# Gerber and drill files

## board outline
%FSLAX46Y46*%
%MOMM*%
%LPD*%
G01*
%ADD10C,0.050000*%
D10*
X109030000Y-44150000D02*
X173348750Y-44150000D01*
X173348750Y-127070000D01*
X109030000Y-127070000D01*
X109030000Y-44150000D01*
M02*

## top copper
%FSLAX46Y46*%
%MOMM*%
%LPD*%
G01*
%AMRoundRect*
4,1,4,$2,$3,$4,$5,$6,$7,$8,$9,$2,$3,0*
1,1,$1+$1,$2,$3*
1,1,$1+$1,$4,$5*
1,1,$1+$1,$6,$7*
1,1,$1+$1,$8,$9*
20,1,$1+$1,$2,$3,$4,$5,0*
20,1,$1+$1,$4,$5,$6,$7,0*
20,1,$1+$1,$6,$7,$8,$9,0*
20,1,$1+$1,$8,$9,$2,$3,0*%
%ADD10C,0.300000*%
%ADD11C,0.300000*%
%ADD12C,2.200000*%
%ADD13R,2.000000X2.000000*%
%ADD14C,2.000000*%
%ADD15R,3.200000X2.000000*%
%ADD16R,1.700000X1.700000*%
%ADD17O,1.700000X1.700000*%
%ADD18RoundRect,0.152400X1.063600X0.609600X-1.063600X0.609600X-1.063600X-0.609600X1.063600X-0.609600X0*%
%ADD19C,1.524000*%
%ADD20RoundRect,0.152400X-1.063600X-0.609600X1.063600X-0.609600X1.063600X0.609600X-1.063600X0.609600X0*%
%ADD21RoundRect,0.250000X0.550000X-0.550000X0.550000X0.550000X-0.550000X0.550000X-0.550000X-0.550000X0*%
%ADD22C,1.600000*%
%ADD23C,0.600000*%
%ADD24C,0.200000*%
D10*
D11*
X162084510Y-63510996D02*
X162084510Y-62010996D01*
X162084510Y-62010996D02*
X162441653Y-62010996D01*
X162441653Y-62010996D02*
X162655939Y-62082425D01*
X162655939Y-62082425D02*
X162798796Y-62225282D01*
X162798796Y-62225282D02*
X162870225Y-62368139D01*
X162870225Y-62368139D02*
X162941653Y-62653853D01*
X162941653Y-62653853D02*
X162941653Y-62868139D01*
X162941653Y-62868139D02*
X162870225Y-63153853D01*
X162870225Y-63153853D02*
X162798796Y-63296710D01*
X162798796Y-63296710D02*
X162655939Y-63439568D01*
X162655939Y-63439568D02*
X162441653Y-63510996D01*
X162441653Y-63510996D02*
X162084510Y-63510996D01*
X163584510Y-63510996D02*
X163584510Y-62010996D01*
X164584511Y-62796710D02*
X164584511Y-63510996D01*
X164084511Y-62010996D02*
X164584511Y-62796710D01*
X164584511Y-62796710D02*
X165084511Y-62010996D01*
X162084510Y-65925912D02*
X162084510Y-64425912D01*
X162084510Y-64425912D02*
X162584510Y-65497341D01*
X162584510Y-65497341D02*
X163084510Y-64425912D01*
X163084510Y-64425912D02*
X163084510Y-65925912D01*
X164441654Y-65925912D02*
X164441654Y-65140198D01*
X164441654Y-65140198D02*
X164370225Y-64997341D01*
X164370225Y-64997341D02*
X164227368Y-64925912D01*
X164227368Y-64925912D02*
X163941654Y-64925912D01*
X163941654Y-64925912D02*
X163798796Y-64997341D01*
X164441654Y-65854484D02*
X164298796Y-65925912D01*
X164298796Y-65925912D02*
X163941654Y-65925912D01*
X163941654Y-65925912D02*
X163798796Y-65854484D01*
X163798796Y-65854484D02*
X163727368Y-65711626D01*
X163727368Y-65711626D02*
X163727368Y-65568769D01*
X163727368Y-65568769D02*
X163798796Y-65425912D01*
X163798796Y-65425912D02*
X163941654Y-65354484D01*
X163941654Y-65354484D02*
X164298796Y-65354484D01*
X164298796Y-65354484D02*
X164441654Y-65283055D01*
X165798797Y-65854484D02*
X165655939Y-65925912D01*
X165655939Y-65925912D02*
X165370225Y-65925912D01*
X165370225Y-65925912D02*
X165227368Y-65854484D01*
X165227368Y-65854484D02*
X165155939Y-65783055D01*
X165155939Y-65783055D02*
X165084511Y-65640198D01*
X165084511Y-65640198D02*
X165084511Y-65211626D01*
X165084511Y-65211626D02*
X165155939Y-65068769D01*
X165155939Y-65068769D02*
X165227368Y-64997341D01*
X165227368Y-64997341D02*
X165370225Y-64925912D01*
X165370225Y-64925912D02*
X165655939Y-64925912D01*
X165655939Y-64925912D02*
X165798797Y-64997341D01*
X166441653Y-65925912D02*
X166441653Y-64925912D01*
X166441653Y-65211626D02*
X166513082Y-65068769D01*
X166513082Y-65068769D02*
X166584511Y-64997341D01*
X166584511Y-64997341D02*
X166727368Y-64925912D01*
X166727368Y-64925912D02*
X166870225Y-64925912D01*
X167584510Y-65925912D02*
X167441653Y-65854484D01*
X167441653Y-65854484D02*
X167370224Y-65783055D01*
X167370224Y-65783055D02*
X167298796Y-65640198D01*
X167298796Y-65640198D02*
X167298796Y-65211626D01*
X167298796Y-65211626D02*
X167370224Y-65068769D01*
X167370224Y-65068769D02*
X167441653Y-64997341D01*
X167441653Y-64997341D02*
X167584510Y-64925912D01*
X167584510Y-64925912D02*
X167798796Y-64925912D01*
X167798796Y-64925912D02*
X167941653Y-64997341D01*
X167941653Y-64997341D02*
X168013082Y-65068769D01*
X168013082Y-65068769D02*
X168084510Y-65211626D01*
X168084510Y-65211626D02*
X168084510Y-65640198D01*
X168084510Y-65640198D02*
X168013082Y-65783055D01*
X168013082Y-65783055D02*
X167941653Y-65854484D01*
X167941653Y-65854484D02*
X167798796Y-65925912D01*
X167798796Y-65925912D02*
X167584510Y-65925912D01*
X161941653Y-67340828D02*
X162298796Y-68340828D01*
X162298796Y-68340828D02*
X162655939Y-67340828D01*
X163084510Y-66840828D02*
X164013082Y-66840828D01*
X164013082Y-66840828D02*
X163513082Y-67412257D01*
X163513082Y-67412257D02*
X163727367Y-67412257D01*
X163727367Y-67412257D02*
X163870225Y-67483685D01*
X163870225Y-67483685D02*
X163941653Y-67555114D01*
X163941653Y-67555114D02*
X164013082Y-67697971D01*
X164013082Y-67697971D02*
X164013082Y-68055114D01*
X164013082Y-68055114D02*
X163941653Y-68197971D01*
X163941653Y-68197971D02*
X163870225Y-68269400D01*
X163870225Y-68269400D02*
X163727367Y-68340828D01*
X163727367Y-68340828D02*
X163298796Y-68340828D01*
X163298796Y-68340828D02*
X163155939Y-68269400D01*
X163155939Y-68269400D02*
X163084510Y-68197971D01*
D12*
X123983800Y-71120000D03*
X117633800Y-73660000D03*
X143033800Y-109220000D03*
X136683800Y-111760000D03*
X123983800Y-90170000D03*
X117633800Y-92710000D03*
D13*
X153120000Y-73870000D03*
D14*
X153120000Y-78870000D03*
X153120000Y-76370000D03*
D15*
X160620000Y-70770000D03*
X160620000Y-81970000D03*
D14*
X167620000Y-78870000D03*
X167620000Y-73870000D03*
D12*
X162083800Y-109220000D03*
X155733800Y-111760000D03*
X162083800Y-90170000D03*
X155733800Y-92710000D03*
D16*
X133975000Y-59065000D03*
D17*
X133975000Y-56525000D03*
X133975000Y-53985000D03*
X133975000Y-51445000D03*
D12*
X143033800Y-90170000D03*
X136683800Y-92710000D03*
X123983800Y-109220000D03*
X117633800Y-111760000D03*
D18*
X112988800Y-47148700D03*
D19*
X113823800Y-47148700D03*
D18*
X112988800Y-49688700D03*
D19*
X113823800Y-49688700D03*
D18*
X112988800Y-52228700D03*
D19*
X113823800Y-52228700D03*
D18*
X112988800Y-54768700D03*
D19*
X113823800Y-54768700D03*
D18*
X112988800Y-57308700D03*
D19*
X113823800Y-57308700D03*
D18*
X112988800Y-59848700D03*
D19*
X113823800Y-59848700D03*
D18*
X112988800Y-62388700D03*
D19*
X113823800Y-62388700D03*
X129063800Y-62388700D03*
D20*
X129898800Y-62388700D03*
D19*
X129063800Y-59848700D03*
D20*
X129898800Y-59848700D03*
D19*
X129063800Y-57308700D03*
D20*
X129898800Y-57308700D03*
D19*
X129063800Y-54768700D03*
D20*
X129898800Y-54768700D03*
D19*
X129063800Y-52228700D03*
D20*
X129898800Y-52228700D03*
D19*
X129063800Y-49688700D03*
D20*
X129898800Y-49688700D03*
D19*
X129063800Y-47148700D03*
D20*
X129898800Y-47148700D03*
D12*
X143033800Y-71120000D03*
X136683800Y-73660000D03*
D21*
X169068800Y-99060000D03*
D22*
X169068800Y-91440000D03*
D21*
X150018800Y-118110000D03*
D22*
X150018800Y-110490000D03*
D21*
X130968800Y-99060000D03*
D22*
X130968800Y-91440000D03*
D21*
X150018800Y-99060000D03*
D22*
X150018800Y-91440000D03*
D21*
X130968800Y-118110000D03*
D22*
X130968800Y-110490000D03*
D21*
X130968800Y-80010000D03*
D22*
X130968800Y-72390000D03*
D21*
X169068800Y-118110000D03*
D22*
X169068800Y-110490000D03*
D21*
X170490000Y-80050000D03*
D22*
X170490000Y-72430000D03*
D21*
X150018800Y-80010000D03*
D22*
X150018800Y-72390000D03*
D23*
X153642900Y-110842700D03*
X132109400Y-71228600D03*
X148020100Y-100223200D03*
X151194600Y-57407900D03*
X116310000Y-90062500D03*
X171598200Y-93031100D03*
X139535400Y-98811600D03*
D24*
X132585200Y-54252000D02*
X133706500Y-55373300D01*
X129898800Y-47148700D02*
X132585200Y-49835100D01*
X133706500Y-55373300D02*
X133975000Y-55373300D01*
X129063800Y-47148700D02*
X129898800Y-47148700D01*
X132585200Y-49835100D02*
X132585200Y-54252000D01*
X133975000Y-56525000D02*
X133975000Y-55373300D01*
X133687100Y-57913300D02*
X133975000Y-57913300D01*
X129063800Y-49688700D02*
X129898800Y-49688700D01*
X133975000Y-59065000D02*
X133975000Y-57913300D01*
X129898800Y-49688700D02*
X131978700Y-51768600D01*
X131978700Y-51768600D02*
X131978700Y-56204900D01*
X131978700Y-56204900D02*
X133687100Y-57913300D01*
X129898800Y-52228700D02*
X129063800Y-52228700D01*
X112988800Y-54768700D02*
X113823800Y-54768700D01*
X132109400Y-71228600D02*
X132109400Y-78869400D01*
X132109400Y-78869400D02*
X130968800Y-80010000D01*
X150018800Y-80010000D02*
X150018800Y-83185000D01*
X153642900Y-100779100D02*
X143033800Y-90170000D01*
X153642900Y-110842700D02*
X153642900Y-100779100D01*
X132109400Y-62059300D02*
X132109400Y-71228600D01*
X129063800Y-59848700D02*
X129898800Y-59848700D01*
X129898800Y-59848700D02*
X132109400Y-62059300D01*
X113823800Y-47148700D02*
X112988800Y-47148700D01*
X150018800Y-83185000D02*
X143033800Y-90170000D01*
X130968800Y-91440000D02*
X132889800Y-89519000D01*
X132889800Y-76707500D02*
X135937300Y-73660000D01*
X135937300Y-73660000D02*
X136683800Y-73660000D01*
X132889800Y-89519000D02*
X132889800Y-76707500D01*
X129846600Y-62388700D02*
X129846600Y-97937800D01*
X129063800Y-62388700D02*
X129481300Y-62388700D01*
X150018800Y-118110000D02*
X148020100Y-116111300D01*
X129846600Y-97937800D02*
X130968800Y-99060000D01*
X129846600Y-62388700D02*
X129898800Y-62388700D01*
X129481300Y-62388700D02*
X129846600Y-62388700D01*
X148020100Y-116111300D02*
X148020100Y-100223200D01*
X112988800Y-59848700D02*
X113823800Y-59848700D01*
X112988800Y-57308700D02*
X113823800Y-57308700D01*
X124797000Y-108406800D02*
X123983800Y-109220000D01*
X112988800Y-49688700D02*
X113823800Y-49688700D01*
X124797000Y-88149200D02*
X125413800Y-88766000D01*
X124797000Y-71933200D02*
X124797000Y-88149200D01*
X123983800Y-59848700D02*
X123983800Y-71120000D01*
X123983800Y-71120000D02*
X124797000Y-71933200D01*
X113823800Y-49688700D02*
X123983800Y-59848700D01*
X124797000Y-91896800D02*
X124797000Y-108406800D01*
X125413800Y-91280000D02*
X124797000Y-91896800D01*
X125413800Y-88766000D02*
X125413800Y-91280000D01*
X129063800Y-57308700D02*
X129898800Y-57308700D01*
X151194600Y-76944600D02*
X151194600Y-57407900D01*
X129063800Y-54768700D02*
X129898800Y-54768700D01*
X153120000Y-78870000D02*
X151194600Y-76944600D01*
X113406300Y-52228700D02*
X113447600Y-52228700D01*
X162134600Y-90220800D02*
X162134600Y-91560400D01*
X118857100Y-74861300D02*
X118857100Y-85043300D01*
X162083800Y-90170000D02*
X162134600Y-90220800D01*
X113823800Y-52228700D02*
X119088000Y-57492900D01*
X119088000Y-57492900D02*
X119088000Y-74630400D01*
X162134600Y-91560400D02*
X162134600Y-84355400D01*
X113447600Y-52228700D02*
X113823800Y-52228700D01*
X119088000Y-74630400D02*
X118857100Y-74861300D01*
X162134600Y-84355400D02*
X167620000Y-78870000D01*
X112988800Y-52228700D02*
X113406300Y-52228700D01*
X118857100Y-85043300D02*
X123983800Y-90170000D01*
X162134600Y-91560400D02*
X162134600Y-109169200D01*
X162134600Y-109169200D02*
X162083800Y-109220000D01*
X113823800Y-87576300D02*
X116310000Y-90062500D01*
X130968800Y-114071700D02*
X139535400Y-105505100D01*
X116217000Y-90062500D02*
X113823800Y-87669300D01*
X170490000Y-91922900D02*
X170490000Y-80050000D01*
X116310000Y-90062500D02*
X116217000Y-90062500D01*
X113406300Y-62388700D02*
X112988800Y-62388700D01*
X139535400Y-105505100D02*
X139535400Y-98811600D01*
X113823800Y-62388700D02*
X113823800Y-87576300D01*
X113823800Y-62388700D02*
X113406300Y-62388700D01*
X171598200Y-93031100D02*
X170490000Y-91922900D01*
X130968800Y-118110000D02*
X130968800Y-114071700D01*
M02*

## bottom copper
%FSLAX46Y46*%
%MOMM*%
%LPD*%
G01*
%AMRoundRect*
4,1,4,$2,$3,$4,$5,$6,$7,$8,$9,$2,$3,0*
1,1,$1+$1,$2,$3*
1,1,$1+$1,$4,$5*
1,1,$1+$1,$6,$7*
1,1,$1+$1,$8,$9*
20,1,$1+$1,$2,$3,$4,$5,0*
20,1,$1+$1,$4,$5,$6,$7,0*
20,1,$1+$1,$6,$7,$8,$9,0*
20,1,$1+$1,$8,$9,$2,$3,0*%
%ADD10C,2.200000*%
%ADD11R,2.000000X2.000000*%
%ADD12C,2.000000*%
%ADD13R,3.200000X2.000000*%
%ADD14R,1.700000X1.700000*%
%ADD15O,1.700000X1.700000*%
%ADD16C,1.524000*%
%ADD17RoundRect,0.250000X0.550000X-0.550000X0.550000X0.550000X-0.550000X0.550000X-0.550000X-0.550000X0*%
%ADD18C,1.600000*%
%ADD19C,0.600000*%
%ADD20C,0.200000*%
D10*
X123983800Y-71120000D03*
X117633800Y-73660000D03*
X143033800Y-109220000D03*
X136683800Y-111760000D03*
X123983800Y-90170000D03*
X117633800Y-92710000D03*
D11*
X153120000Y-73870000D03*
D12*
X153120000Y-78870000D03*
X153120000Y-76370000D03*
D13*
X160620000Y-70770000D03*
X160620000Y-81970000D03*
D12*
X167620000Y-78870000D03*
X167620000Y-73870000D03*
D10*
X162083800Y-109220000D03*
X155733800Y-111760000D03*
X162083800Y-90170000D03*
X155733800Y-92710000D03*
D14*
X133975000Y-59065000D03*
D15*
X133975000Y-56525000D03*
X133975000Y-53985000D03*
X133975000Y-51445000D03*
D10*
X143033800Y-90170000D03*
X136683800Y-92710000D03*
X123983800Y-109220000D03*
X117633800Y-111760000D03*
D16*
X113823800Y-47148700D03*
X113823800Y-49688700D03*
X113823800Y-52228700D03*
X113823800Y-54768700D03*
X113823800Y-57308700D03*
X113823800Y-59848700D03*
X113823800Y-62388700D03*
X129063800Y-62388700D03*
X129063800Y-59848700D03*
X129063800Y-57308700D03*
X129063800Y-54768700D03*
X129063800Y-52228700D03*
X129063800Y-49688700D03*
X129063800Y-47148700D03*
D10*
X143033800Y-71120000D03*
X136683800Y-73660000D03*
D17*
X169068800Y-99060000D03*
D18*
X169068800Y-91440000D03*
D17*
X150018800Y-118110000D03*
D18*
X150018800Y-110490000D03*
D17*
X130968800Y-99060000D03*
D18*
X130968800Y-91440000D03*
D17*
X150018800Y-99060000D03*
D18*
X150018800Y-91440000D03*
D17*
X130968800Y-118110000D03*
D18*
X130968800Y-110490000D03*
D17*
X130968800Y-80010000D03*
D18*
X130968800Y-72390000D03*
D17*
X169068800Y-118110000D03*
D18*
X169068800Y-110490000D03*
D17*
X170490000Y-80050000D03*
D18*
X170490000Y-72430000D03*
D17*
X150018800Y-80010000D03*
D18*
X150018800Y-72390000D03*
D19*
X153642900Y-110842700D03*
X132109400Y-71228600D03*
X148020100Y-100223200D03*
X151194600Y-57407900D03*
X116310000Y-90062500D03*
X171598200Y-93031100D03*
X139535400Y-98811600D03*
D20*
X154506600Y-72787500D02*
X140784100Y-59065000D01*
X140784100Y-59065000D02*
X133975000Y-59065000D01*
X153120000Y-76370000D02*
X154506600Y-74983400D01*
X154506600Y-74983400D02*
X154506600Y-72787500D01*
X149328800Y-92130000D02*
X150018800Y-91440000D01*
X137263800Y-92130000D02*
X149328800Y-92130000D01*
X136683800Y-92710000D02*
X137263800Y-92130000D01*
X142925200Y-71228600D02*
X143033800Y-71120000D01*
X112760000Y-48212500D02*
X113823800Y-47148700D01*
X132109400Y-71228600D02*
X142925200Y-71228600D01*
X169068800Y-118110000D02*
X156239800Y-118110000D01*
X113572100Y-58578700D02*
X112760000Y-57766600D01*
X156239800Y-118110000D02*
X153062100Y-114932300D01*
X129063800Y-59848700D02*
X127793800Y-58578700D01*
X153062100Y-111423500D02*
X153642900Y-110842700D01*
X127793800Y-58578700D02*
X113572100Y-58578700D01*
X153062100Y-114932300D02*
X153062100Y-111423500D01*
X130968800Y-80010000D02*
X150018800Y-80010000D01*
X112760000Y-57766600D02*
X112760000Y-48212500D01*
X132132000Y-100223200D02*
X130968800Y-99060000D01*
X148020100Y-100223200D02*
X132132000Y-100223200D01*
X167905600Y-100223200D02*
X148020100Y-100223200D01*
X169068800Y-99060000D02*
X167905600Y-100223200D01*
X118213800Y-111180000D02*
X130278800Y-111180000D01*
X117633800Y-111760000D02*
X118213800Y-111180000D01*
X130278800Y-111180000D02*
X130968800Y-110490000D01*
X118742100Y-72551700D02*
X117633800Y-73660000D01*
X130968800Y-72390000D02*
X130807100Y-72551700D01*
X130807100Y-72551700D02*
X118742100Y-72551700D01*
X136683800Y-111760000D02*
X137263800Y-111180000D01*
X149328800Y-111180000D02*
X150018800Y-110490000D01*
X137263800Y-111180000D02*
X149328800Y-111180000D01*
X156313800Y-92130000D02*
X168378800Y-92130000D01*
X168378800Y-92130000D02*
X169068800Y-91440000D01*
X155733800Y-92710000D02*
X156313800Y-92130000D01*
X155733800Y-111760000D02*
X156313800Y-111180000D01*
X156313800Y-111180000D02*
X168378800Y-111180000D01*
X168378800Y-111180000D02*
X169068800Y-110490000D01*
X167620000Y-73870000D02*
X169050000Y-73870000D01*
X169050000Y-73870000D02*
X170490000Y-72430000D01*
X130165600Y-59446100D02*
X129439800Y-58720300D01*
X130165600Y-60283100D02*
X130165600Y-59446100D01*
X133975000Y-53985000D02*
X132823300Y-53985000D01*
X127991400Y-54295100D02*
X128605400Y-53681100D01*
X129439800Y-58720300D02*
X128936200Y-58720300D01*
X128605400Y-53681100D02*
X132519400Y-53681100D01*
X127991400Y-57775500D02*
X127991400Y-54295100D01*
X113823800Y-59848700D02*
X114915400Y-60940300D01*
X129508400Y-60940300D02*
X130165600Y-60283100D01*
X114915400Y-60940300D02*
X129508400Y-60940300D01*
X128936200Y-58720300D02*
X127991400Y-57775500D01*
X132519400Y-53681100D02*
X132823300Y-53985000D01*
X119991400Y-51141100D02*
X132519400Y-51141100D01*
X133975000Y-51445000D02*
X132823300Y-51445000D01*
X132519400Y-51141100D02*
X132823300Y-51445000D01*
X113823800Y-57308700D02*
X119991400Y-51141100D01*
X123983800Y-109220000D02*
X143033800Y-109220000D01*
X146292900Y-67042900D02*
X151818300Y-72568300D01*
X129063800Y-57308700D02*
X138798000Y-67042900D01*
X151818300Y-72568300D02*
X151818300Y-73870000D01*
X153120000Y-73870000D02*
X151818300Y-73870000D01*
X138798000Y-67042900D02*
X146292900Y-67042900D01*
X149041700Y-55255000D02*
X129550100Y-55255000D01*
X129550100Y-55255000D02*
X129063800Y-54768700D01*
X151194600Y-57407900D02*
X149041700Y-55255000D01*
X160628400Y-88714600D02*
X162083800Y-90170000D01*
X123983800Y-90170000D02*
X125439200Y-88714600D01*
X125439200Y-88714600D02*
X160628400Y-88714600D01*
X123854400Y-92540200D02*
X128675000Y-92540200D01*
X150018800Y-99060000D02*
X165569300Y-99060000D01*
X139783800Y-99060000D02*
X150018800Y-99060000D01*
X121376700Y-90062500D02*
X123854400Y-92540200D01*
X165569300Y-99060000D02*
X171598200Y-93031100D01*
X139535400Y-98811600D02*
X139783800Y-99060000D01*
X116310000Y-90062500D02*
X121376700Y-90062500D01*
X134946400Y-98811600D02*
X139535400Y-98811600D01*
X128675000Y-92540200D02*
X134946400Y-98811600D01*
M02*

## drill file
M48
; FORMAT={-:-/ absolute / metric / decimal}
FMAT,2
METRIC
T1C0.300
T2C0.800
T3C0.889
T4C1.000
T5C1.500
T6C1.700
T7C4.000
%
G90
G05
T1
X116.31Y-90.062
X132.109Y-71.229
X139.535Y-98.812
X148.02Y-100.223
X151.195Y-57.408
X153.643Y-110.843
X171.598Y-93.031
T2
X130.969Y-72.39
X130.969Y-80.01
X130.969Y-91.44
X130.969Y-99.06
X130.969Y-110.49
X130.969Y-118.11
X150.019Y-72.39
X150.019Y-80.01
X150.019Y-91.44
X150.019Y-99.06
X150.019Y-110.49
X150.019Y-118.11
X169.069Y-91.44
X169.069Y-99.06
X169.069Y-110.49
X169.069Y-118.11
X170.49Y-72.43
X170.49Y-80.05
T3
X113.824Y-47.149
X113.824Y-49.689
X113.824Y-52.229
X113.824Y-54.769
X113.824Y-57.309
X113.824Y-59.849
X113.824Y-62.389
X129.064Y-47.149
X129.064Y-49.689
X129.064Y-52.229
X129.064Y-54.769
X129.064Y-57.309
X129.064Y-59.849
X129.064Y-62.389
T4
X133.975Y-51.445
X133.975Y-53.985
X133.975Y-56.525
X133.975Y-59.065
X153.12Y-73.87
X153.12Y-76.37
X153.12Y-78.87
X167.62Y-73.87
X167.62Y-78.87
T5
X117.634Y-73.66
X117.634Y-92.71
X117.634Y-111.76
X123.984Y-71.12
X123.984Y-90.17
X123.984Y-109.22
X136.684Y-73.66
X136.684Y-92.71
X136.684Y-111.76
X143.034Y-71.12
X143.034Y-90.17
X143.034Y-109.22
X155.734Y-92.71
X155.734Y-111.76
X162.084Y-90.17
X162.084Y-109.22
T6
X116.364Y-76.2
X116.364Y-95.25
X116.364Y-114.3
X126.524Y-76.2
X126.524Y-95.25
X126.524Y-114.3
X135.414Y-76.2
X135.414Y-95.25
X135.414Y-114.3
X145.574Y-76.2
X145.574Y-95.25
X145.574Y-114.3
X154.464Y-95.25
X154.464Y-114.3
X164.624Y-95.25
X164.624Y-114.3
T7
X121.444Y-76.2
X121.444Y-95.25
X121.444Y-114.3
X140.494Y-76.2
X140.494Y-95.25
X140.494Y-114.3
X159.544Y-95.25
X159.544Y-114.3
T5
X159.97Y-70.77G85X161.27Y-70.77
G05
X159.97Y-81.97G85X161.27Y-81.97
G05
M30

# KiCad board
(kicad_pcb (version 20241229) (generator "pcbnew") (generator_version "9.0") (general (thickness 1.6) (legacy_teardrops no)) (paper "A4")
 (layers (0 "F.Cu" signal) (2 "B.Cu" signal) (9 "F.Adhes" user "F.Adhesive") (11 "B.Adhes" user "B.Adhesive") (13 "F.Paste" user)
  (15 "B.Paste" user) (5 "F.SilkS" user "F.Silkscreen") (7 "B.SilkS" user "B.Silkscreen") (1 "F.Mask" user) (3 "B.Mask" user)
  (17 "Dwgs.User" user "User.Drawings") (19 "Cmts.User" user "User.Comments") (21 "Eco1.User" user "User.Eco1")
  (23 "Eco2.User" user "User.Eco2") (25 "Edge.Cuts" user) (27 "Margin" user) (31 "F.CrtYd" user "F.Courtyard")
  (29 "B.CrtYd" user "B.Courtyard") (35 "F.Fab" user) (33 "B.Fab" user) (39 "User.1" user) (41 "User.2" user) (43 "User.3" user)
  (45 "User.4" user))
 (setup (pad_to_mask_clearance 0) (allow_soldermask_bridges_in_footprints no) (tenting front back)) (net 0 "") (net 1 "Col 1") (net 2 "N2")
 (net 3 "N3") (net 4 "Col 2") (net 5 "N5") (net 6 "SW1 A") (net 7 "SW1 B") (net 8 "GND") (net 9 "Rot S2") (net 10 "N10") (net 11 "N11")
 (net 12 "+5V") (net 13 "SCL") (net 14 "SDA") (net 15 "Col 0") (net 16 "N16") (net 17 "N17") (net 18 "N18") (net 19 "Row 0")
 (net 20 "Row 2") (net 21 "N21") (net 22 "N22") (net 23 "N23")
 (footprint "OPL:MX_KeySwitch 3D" (layer "F.Cu") (at 123.9838 71.12)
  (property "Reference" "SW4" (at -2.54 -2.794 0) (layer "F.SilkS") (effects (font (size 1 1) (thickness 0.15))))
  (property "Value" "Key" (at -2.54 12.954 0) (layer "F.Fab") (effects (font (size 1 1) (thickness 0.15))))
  (pad "" np_thru_hole circle (at -7.62 5.08) (size 1.7 1.7) (drill 1.7) (layers "*.Cu" "*.Mask"))
  (pad "" np_thru_hole circle (at -2.54 5.08) (size 4 4) (drill 4) (layers "*.Cu" "*.Mask"))
  (pad "" np_thru_hole circle (at 2.54 5.08) (size 1.7 1.7) (drill 1.7) (layers "*.Cu" "*.Mask"))
  (pad "1" thru_hole circle (at 0 0) (size 2.2 2.2) (drill 1.5) (layers "*.Cu" "*.Mask") (remove_unused_layers no) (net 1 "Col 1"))
  (pad "2" thru_hole circle (at -6.35 2.54) (size 2.2 2.2) (drill 1.5) (layers "*.Cu" "*.Mask") (remove_unused_layers no) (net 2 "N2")))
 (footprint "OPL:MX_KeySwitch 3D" (layer "F.Cu") (at 143.0338 109.22)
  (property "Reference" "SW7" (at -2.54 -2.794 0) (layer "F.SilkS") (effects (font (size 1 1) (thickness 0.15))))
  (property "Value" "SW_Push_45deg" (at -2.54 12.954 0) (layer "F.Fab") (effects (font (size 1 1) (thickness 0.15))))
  (pad "" np_thru_hole circle (at -7.62 5.08) (size 1.7 1.7) (drill 1.7) (layers "*.Cu" "*.Mask"))
  (pad "" np_thru_hole circle (at -2.54 5.08) (size 4 4) (drill 4) (layers "*.Cu" "*.Mask"))
  (pad "" np_thru_hole circle (at 2.54 5.08) (size 1.7 1.7) (drill 1.7) (layers "*.Cu" "*.Mask"))
  (pad "1" thru_hole circle (at 0 0) (size 2.2 2.2) (drill 1.5) (layers "*.Cu" "*.Mask") (remove_unused_layers no) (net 1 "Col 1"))
  (pad "2" thru_hole circle (at -6.35 2.54) (size 2.2 2.2) (drill 1.5) (layers "*.Cu" "*.Mask") (remove_unused_layers no) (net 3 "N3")))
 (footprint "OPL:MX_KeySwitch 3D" (layer "F.Cu") (at 123.9838 90.17)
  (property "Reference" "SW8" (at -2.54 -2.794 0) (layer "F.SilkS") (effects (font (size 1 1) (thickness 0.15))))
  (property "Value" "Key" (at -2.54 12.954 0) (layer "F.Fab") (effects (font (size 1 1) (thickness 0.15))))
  (pad "" np_thru_hole circle (at -7.62 5.08) (size 1.7 1.7) (drill 1.7) (layers "*.Cu" "*.Mask"))
  (pad "" np_thru_hole circle (at -2.54 5.08) (size 4 4) (drill 4) (layers "*.Cu" "*.Mask"))
  (pad "" np_thru_hole circle (at 2.54 5.08) (size 1.7 1.7) (drill 1.7) (layers "*.Cu" "*.Mask"))
  (pad "1" thru_hole circle (at 0 0) (size 2.2 2.2) (drill 1.5) (layers "*.Cu" "*.Mask") (remove_unused_layers no) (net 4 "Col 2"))
  (pad "2" thru_hole circle (at -6.35 2.54) (size 2.2 2.2) (drill 1.5) (layers "*.Cu" "*.Mask") (remove_unused_layers no) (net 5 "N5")))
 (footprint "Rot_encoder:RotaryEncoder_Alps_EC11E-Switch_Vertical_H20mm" (layer "F.Cu") (at 153.12 73.87)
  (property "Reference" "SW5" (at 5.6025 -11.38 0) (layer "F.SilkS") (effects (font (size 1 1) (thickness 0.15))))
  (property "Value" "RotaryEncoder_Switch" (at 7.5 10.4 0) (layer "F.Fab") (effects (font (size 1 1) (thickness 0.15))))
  (pad "A" thru_hole rect (at 0 0) (size 2 2) (drill 1) (layers "*.Cu" "*.Mask") (remove_unused_layers no) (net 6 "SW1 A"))
  (pad "B" thru_hole circle (at 0 5) (size 2 2) (drill 1) (layers "*.Cu" "*.Mask") (remove_unused_layers no) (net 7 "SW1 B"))
  (pad "C" thru_hole circle (at 0 2.5) (size 2 2) (drill 1) (layers "*.Cu" "*.Mask") (remove_unused_layers no) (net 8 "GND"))
  (pad "MP" thru_hole rect (at 7.5 -3.1) (size 3.2 2) (drill oval 2.8 1.5) (layers "*.Cu" "*.Mask") (remove_unused_layers no))
  (pad "MP" thru_hole rect (at 7.5 8.1) (size 3.2 2) (drill oval 2.8 1.5) (layers "*.Cu" "*.Mask") (remove_unused_layers no))
  (pad "S1" thru_hole circle (at 14.5 5) (size 2 2) (drill 1) (layers "*.Cu" "*.Mask") (remove_unused_layers no) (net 4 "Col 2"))
  (pad "S2" thru_hole circle (at 14.5 0) (size 2 2) (drill 1) (layers "*.Cu" "*.Mask") (remove_unused_layers no) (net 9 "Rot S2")))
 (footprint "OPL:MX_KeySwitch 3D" (layer "F.Cu") (at 162.0838 109.22)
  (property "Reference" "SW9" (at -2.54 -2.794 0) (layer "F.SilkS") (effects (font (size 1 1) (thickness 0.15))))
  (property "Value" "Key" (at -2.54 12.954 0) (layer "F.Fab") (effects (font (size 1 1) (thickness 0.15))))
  (pad "" np_thru_hole circle (at -7.62 5.08) (size 1.7 1.7) (drill 1.7) (layers "*.Cu" "*.Mask"))
  (pad "" np_thru_hole circle (at -2.54 5.08) (size 4 4) (drill 4) (layers "*.Cu" "*.Mask"))
  (pad "" np_thru_hole circle (at 2.54 5.08) (size 1.7 1.7) (drill 1.7) (layers "*.Cu" "*.Mask"))
  (pad "1" thru_hole circle (at 0 0) (size 2.2 2.2) (drill 1.5) (layers "*.Cu" "*.Mask") (remove_unused_layers no) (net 4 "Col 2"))
  (pad "2" thru_hole circle (at -6.35 2.54) (size 2.2 2.2) (drill 1.5) (layers "*.Cu" "*.Mask") (remove_unused_layers no) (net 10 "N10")))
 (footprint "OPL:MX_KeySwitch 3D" (layer "F.Cu") (at 162.0838 90.17)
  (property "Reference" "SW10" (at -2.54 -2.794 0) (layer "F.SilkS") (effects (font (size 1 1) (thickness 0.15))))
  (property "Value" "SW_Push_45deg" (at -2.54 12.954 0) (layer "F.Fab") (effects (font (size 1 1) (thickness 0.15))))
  (pad "" np_thru_hole circle (at -7.62 5.08) (size 1.7 1.7) (drill 1.7) (layers "*.Cu" "*.Mask"))
  (pad "" np_thru_hole circle (at -2.54 5.08) (size 4 4) (drill 4) (layers "*.Cu" "*.Mask"))
  (pad "" np_thru_hole circle (at 2.54 5.08) (size 1.7 1.7) (drill 1.7) (layers "*.Cu" "*.Mask"))
  (pad "1" thru_hole circle (at 0 0) (size 2.2 2.2) (drill 1.5) (layers "*.Cu" "*.Mask") (remove_unused_layers no) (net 4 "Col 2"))
  (pad "2" thru_hole circle (at -6.35 2.54) (size 2.2 2.2) (drill 1.5) (layers "*.Cu" "*.Mask") (remove_unused_layers no) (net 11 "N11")))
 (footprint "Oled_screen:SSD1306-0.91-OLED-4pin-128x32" (layer "F.Cu") (at 170.475 61.255 180)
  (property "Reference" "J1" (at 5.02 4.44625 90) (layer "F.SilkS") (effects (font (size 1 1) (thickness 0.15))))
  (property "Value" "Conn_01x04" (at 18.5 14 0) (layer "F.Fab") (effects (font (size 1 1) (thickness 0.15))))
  (pad "1" thru_hole rect (at 36.5 2.19 180) (size 1.7 1.7) (drill 1) (layers "*.Cu" "*.Mask") (remove_unused_layers no) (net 8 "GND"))
  (pad "2" thru_hole oval (at 36.5 4.73 180) (size 1.7 1.7) (drill 1) (layers "*.Cu" "*.Mask") (remove_unused_layers no) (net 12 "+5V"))
  (pad "3" thru_hole oval (at 36.5 7.27 180) (size 1.7 1.7) (drill 1) (layers "*.Cu" "*.Mask") (remove_unused_layers no) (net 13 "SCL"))
  (pad "4" thru_hole oval (at 36.5 9.81 180) (size 1.7 1.7) (drill 1) (layers "*.Cu" "*.Mask") (remove_unused_layers no) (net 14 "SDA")))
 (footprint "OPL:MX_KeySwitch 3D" (layer "F.Cu") (at 143.0338 90.17)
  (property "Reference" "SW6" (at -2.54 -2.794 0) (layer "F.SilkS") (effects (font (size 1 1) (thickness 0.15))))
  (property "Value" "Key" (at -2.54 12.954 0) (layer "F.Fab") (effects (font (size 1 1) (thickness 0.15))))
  (pad "" np_thru_hole circle (at -7.62 5.08) (size 1.7 1.7) (drill 1.7) (layers "*.Cu" "*.Mask"))
  (pad "" np_thru_hole circle (at -2.54 5.08) (size 4 4) (drill 4) (layers "*.Cu" "*.Mask"))
  (pad "" np_thru_hole circle (at 2.54 5.08) (size 1.7 1.7) (drill 1.7) (layers "*.Cu" "*.Mask"))
  (pad "1" thru_hole circle (at 0 0) (size 2.2 2.2) (drill 1.5) (layers "*.Cu" "*.Mask") (remove_unused_layers no) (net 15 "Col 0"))
  (pad "2" thru_hole circle (at -6.35 2.54) (size 2.2 2.2) (drill 1.5) (layers "*.Cu" "*.Mask") (remove_unused_layers no) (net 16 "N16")))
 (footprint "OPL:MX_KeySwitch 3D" (layer "F.Cu") (at 123.9838 109.22)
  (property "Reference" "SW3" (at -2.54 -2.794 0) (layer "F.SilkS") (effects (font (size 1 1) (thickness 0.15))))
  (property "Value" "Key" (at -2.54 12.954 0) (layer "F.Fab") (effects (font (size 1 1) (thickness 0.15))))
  (pad "" np_thru_hole circle (at -7.62 5.08) (size 1.7 1.7) (drill 1.7) (layers "*.Cu" "*.Mask"))
  (pad "" np_thru_hole circle (at -2.54 5.08) (size 4 4) (drill 4) (layers "*.Cu" "*.Mask"))
  (pad "" np_thru_hole circle (at 2.54 5.08) (size 1.7 1.7) (drill 1.7) (layers "*.Cu" "*.Mask"))
  (pad "1" thru_hole circle (at 0 0) (size 2.2 2.2) (drill 1.5) (layers "*.Cu" "*.Mask") (remove_unused_layers no) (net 1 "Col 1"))
  (pad "2" thru_hole circle (at -6.35 2.54) (size 2.2 2.2) (drill 1.5) (layers "*.Cu" "*.Mask") (remove_unused_layers no) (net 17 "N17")))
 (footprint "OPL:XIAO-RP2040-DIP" (layer "F.Cu") (at 121.4438 54.7687)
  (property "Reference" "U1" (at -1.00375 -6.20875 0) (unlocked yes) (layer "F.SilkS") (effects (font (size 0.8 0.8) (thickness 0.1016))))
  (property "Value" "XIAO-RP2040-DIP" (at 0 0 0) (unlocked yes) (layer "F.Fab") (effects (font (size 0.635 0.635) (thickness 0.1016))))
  (pad "1" smd roundrect (at -8.455 -7.62 180) (size 2.432 1.524) (layers "F.Cu" "F.Mask") (roundrect_rratio 0.1) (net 15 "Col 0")
   (thermal_bridge_angle 45))
  (pad "1" thru_hole circle (at -7.62 -7.62 180) (size 1.524 1.524) (drill 0.889) (layers "*.Cu" "*.Mask") (remove_unused_layers no)
   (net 15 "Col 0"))
  (pad "2" smd roundrect (at -8.455 -5.08 180) (size 2.432 1.524) (layers "F.Cu" "F.Mask") (roundrect_rratio 0.1) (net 1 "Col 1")
   (thermal_bridge_angle 45))
  (pad "2" thru_hole circle (at -7.62 -5.08 180) (size 1.524 1.524) (drill 0.889) (layers "*.Cu" "*.Mask") (remove_unused_layers no)
   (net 1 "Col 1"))
  (pad "3" smd roundrect (at -8.455 -2.54 180) (size 2.432 1.524) (layers "F.Cu" "F.Mask") (roundrect_rratio 0.1) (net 4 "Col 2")
   (thermal_bridge_angle 45))
  (pad "3" thru_hole circle (at -7.62 -2.54 180) (size 1.524 1.524) (drill 0.889) (layers "*.Cu" "*.Mask") (remove_unused_layers no)
   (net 4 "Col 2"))
  (pad "4" smd roundrect (at -8.455 0 180) (size 2.432 1.524) (layers "F.Cu" "F.Mask") (roundrect_rratio 0.1) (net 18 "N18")
   (thermal_bridge_angle 45))
  (pad "4" thru_hole circle (at -7.62 0 180) (size 1.524 1.524) (drill 0.889) (layers "*.Cu" "*.Mask") (remove_unused_layers no)
   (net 18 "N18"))
  (pad "5" smd roundrect (at -8.455 2.54 180) (size 2.432 1.524) (layers "F.Cu" "F.Mask") (roundrect_rratio 0.1) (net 14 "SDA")
   (thermal_bridge_angle 45))
  (pad "5" thru_hole circle (at -7.62 2.54 180) (size 1.524 1.524) (drill 0.889) (layers "*.Cu" "*.Mask") (remove_unused_layers no)
   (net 14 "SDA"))
  (pad "6" smd roundrect (at -8.455 5.08 180) (size 2.432 1.524) (layers "F.Cu" "F.Mask") (roundrect_rratio 0.1) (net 13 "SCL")
   (thermal_bridge_angle 45))
  (pad "6" thru_hole circle (at -7.62 5.08 180) (size 1.524 1.524) (drill 0.889) (layers "*.Cu" "*.Mask") (remove_unused_layers no)
   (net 13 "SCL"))
  (pad "7" smd roundrect (at -8.455 7.62 180) (size 2.432 1.524) (layers "F.Cu" "F.Mask") (roundrect_rratio 0.1) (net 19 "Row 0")
   (thermal_bridge_angle 45))
  (pad "7" thru_hole circle (at -7.62 7.62 180) (size 1.524 1.524) (drill 0.889) (layers "*.Cu" "*.Mask") (remove_unused_layers no)
   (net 19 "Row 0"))
  (pad "8" thru_hole circle (at 7.62 7.62) (size 1.524 1.524) (drill 0.889) (layers "*.Cu" "*.Mask") (remove_unused_layers no)
   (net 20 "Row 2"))
  (pad "8" smd roundrect (at 8.455 7.62) (size 2.432 1.524) (layers "F.Cu" "F.Mask") (roundrect_rratio 0.1) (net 20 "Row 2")
   (thermal_bridge_angle 45))
  (pad "9" thru_hole circle (at 7.62 5.08) (size 1.524 1.524) (drill 0.889) (layers "*.Cu" "*.Mask") (remove_unused_layers no)
   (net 15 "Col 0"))
  (pad "9" smd roundrect (at 8.455 5.08) (size 2.432 1.524) (layers "F.Cu" "F.Mask") (roundrect_rratio 0.1) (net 15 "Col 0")
   (thermal_bridge_angle 45))
  (pad "10" thru_hole circle (at 7.62 2.54) (size 1.524 1.524) (drill 0.889) (layers "*.Cu" "*.Mask") (remove_unused_layers no)
   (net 6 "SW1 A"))
  (pad "10" smd roundrect (at 8.455 2.54) (size 2.432 1.524) (layers "F.Cu" "F.Mask") (roundrect_rratio 0.1) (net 6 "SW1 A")
   (thermal_bridge_angle 45))
  (pad "11" thru_hole circle (at 7.62 0) (size 1.524 1.524) (drill 0.889) (layers "*.Cu" "*.Mask") (remove_unused_layers no) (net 7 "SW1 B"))
  (pad "11" smd roundrect (at 8.455 0) (size 2.432 1.524) (layers "F.Cu" "F.Mask") (roundrect_rratio 0.1) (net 7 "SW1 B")
   (thermal_bridge_angle 45))
  (pad "12" thru_hole circle (at 7.62 -2.54) (size 1.524 1.524) (drill 0.889) (layers "*.Cu" "*.Mask") (remove_unused_layers no)
   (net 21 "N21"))
  (pad "12" smd roundrect (at 8.455 -2.54) (size 2.432 1.524) (layers "F.Cu" "F.Mask") (roundrect_rratio 0.1) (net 21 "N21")
   (thermal_bridge_angle 45))
  (pad "13" thru_hole circle (at 7.62 -5.08) (size 1.524 1.524) (drill 0.889) (layers "*.Cu" "*.Mask") (remove_unused_layers no)
   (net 8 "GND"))
  (pad "13" smd roundrect (at 8.455 -5.08) (size 2.432 1.524) (layers "F.Cu" "F.Mask") (roundrect_rratio 0.1) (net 8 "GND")
   (thermal_bridge_angle 45))
  (pad "14" thru_hole circle (at 7.62 -7.62) (size 1.524 1.524) (drill 0.889) (layers "*.Cu" "*.Mask") (remove_unused_layers no)
   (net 12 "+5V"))
  (pad "14" smd roundrect (at 8.455 -7.62) (size 2.432 1.524) (layers "F.Cu" "F.Mask") (roundrect_rratio 0.1) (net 12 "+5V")
   (thermal_bridge_angle 45)))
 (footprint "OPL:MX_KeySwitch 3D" (layer "F.Cu") (at 143.0338 71.12)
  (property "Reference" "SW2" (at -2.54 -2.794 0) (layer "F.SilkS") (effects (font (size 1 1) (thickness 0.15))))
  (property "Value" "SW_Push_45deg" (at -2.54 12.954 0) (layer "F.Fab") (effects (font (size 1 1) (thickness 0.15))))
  (pad "" np_thru_hole circle (at -7.62 5.08) (size 1.7 1.7) (drill 1.7) (layers "*.Cu" "*.Mask"))
  (pad "" np_thru_hole circle (at -2.54 5.08) (size 4 4) (drill 4) (layers "*.Cu" "*.Mask"))
  (pad "" np_thru_hole circle (at 2.54 5.08) (size 1.7 1.7) (drill 1.7) (layers "*.Cu" "*.Mask"))
  (pad "1" thru_hole circle (at 0 0) (size 2.2 2.2) (drill 1.5) (layers "*.Cu" "*.Mask") (remove_unused_layers no) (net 15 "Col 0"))
  (pad "2" thru_hole circle (at -6.35 2.54) (size 2.2 2.2) (drill 1.5) (layers "*.Cu" "*.Mask") (remove_unused_layers no) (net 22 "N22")))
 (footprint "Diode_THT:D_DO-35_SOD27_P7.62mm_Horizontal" (layer "B.Cu") (at 169.0688 99.06 90)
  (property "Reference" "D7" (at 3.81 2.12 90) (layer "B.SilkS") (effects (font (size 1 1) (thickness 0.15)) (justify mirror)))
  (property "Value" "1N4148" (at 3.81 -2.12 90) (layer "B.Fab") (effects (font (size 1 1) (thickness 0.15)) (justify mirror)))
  (pad "1" thru_hole roundrect (at 0 0 90) (size 1.6 1.6) (drill 0.8) (layers "*.Cu" "*.Mask") (remove_unused_layers no)
   (roundrect_rratio 0.15625) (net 20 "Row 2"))
  (pad "2" thru_hole circle (at 7.62 0 90) (size 1.6 1.6) (drill 0.8) (layers "*.Cu" "*.Mask") (remove_unused_layers no) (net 11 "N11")))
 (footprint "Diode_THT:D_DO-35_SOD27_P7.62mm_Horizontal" (layer "B.Cu") (at 150.0188 118.11 90)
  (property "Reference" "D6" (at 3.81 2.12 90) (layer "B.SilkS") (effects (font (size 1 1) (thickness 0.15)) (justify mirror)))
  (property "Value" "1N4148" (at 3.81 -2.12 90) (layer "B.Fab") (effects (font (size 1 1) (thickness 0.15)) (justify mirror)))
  (pad "1" thru_hole roundrect (at 0 0 90) (size 1.6 1.6) (drill 0.8) (layers "*.Cu" "*.Mask") (remove_unused_layers no)
   (roundrect_rratio 0.15625) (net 20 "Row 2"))
  (pad "2" thru_hole circle (at 7.62 0 90) (size 1.6 1.6) (drill 0.8) (layers "*.Cu" "*.Mask") (remove_unused_layers no) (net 3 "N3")))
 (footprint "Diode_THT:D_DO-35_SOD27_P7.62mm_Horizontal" (layer "B.Cu") (at 130.9688 99.06 90)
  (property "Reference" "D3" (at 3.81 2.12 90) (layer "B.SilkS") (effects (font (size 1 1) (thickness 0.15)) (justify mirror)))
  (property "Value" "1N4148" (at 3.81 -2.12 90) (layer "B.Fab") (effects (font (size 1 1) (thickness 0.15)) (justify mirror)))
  (pad "1" thru_hole roundrect (at 0 0 90) (size 1.6 1.6) (drill 0.8) (layers "*.Cu" "*.Mask") (remove_unused_layers no)
   (roundrect_rratio 0.15625) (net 20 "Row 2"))
  (pad "2" thru_hole circle (at 7.62 0 90) (size 1.6 1.6) (drill 0.8) (layers "*.Cu" "*.Mask") (remove_unused_layers no) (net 22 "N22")))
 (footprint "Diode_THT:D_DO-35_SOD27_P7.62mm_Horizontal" (layer "B.Cu") (at 150.0188 99.06 90)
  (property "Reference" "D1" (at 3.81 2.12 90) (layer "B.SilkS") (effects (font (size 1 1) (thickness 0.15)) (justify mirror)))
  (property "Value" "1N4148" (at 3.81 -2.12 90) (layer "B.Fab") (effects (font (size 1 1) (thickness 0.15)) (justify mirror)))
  (pad "1" thru_hole roundrect (at 0 0 90) (size 1.6 1.6) (drill 0.8) (layers "*.Cu" "*.Mask") (remove_unused_layers no)
   (roundrect_rratio 0.15625) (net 19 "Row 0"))
  (pad "2" thru_hole circle (at 7.62 0 90) (size 1.6 1.6) (drill 0.8) (layers "*.Cu" "*.Mask") (remove_unused_layers no) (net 16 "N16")))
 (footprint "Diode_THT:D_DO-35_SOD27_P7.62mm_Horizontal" (layer "B.Cu") (at 130.9688 118.11 90)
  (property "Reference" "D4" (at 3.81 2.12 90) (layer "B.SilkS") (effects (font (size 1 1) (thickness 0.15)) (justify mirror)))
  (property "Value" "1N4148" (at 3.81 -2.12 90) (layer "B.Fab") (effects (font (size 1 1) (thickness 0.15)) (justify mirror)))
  (pad "1" thru_hole roundrect (at 0 0 90) (size 1.6 1.6) (drill 0.8) (layers "*.Cu" "*.Mask") (remove_unused_layers no)
   (roundrect_rratio 0.15625) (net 19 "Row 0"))
  (pad "2" thru_hole circle (at 7.62 0 90) (size 1.6 1.6) (drill 0.8) (layers "*.Cu" "*.Mask") (remove_unused_layers no) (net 17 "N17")))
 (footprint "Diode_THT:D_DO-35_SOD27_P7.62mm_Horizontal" (layer "B.Cu") (at 130.9688 80.01 90)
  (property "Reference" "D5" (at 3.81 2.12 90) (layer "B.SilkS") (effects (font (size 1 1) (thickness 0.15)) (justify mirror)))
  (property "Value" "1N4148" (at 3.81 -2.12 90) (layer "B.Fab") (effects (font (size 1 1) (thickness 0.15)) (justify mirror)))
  (pad "1" thru_hole roundrect (at 0 0 90) (size 1.6 1.6) (drill 0.8) (layers "*.Cu" "*.Mask") (remove_unused_layers no)
   (roundrect_rratio 0.15625) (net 15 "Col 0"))
  (pad "2" thru_hole circle (at 7.62 0 90) (size 1.6 1.6) (drill 0.8) (layers "*.Cu" "*.Mask") (remove_unused_layers no) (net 2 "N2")))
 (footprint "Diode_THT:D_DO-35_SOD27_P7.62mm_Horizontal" (layer "B.Cu") (at 169.0688 118.11 90)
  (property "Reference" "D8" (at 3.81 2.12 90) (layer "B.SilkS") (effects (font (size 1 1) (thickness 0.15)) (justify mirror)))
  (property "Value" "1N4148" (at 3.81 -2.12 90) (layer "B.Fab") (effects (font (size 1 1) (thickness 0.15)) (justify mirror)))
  (pad "1" thru_hole roundrect (at 0 0 90) (size 1.6 1.6) (drill 0.8) (layers "*.Cu" "*.Mask") (remove_unused_layers no)
   (roundrect_rratio 0.15625) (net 15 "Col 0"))
  (pad "2" thru_hole circle (at 7.62 0 90) (size 1.6 1.6) (drill 0.8) (layers "*.Cu" "*.Mask") (remove_unused_layers no) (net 10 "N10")))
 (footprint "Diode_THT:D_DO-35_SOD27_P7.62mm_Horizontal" (layer "B.Cu") (at 170.49 80.05 90)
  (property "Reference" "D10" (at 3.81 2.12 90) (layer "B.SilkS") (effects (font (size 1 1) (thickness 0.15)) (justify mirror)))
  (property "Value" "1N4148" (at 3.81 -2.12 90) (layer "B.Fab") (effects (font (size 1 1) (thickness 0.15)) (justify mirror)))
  (pad "1" thru_hole roundrect (at 0 0 90) (size 1.6 1.6) (drill 0.8) (layers "*.Cu" "*.Mask") (remove_unused_layers no)
   (roundrect_rratio 0.15625) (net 19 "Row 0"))
  (pad "2" thru_hole circle (at 7.62 0 90) (size 1.6 1.6) (drill 0.8) (layers "*.Cu" "*.Mask") (remove_unused_layers no) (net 9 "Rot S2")))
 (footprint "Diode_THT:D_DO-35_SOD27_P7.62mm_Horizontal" (layer "B.Cu") (at 150.0188 80.01 90)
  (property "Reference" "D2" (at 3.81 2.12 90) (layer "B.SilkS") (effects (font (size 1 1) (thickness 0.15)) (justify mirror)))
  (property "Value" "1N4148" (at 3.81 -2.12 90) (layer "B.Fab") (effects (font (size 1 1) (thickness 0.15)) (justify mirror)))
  (pad "1" thru_hole roundrect (at 0 0 90) (size 1.6 1.6) (drill 0.8) (layers "*.Cu" "*.Mask") (remove_unused_layers no)
   (roundrect_rratio 0.15625) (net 15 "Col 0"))
  (pad "2" thru_hole circle (at 7.62 0 90) (size 1.6 1.6) (drill 0.8) (layers "*.Cu" "*.Mask") (remove_unused_layers no) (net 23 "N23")))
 (gr_rect (start 109.03 44.15) (end 173.34875 127.07) (stroke (width 0.05) (type default)) (fill no) (layer "Edge.Cuts"))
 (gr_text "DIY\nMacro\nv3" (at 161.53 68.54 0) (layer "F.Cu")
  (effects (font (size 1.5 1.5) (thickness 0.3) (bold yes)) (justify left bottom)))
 (segment (start 132.5852 54.252) (end 133.7065 55.3733) (width 0.2) (layer "F.Cu") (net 12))
 (segment (start 129.8988 47.1487) (end 132.5852 49.8351) (width 0.2) (layer "F.Cu") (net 12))
 (segment (start 133.7065 55.3733) (end 133.975 55.3733) (width 0.2) (layer "F.Cu") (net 12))
 (segment (start 129.0638 47.1487) (end 129.8988 47.1487) (width 0.2) (layer "F.Cu") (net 12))
 (segment (start 132.5852 49.8351) (end 132.5852 54.252) (width 0.2) (layer "F.Cu") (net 12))
 (segment (start 133.975 56.525) (end 133.975 55.3733) (width 0.2) (layer "F.Cu") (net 12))
 (segment (start 133.6871 57.9133) (end 133.975 57.9133) (width 0.2) (layer "F.Cu") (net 8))
 (segment (start 129.0638 49.6887) (end 129.8988 49.6887) (width 0.2) (layer "F.Cu") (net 8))
 (segment (start 133.975 59.065) (end 133.975 57.9133) (width 0.2) (layer "F.Cu") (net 8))
 (segment (start 129.8988 49.6887) (end 131.9787 51.7686) (width 0.2) (layer "F.Cu") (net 8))
 (segment (start 131.9787 51.7686) (end 131.9787 56.2049) (width 0.2) (layer "F.Cu") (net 8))
 (segment (start 131.9787 56.2049) (end 133.6871 57.9133) (width 0.2) (layer "F.Cu") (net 8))
 (segment (start 154.5066 72.7875) (end 140.7841 59.065) (width 0.2) (layer "B.Cu") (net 8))
 (segment (start 140.7841 59.065) (end 133.975 59.065) (width 0.2) (layer "B.Cu") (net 8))
 (segment (start 153.12 76.37) (end 154.5066 74.9834) (width 0.2) (layer "B.Cu") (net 8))
 (segment (start 154.5066 74.9834) (end 154.5066 72.7875) (width 0.2) (layer "B.Cu") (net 8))
 (segment (start 129.8988 52.2287) (end 129.0638 52.2287) (width 0.2) (layer "F.Cu") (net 21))
 (segment (start 149.3288 92.13) (end 150.0188 91.44) (width 0.2) (layer "B.Cu") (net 16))
 (segment (start 137.2638 92.13) (end 149.3288 92.13) (width 0.2) (layer "B.Cu") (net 16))
 (segment (start 136.6838 92.71) (end 137.2638 92.13) (width 0.2) (layer "B.Cu") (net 16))
 (segment (start 112.9888 54.7687) (end 113.8238 54.7687) (width 0.2) (layer "F.Cu") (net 18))
 (segment (start 132.1094 71.2286) (end 132.1094 78.8694) (width 0.2) (layer "F.Cu") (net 15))
 (segment (start 132.1094 78.8694) (end 130.9688 80.01) (width 0.2) (layer "F.Cu") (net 15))
 (segment (start 150.0188 80.01) (end 150.0188 83.185) (width 0.2) (layer "F.Cu") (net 15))
 (segment (start 153.6429 100.7791) (end 143.0338 90.17) (width 0.2) (layer "F.Cu") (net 15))
 (segment (start 153.6429 110.8427) (end 153.6429 100.7791) (width 0.2) (layer "F.Cu") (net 15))
 (segment (start 132.1094 62.0593) (end 132.1094 71.2286) (width 0.2) (layer "F.Cu") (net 15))
 (segment (start 129.0638 59.8487) (end 129.8988 59.8487) (width 0.2) (layer "F.Cu") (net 15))
 (segment (start 129.8988 59.8487) (end 132.1094 62.0593) (width 0.2) (layer "F.Cu") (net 15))
 (segment (start 113.8238 47.1487) (end 112.9888 47.1487) (width 0.2) (layer "F.Cu") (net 15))
 (segment (start 150.0188 83.185) (end 143.0338 90.17) (width 0.2) (layer "F.Cu") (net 15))
 (via (at 153.6429 110.8427) (size 0.6) (drill 0.3) (layers "F.Cu" "B.Cu") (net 15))
 (via (at 132.1094 71.2286) (size 0.6) (drill 0.3) (layers "F.Cu" "B.Cu") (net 15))
 (segment (start 142.9252 71.2286) (end 143.0338 71.12) (width 0.2) (layer "B.Cu") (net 15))
 (segment (start 112.76 48.2125) (end 113.8238 47.1487) (width 0.2) (layer "B.Cu") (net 15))
 (segment (start 132.1094 71.2286) (end 142.9252 71.2286) (width 0.2) (layer "B.Cu") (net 15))
 (segment (start 169.0688 118.11) (end 156.2398 118.11) (width 0.2) (layer "B.Cu") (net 15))
 (segment (start 113.5721 58.5787) (end 112.76 57.7666) (width 0.2) (layer "B.Cu") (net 15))
 (segment (start 156.2398 118.11) (end 153.0621 114.9323) (width 0.2) (layer "B.Cu") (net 15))
 (segment (start 129.0638 59.8487) (end 127.7938 58.5787) (width 0.2) (layer "B.Cu") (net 15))
 (segment (start 153.0621 111.4235) (end 153.6429 110.8427) (width 0.2) (layer "B.Cu") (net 15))
 (segment (start 127.7938 58.5787) (end 113.5721 58.5787) (width 0.2) (layer "B.Cu") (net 15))
 (segment (start 153.0621 114.9323) (end 153.0621 111.4235) (width 0.2) (layer "B.Cu") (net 15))
 (segment (start 130.9688 80.01) (end 150.0188 80.01) (width 0.2) (layer "B.Cu") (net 15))
 (segment (start 112.76 57.7666) (end 112.76 48.2125) (width 0.2) (layer "B.Cu") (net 15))
 (segment (start 130.9688 91.44) (end 132.8898 89.519) (width 0.2) (layer "F.Cu") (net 22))
 (segment (start 132.8898 76.7075) (end 135.9373 73.66) (width 0.2) (layer "F.Cu") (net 22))
 (segment (start 135.9373 73.66) (end 136.6838 73.66) (width 0.2) (layer "F.Cu") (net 22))
 (segment (start 132.8898 89.519) (end 132.8898 76.7075) (width 0.2) (layer "F.Cu") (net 22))
 (segment (start 129.8466 62.3887) (end 129.8466 97.9378) (width 0.2) (layer "F.Cu") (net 20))
 (segment (start 129.0638 62.3887) (end 129.4813 62.3887) (width 0.2) (layer "F.Cu") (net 20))
 (segment (start 150.0188 118.11) (end 148.0201 116.1113) (width 0.2) (layer "F.Cu") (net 20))
 (segment (start 129.8466 97.9378) (end 130.9688 99.06) (width 0.2) (layer "F.Cu") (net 20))
 (segment (start 129.8466 62.3887) (end 129.8988 62.3887) (width 0.2) (layer "F.Cu") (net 20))
 (segment (start 129.4813 62.3887) (end 129.8466 62.3887) (width 0.2) (layer "F.Cu") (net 20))
 (segment (start 148.0201 116.1113) (end 148.0201 100.2232) (width 0.2) (layer "F.Cu") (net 20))
 (via (at 148.0201 100.2232) (size 0.6) (drill 0.3) (layers "F.Cu" "B.Cu") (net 20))
 (segment (start 132.132 100.2232) (end 130.9688 99.06) (width 0.2) (layer "B.Cu") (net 20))
 (segment (start 148.0201 100.2232) (end 132.132 100.2232) (width 0.2) (layer "B.Cu") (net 20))
 (segment (start 167.9056 100.2232) (end 148.0201 100.2232) (width 0.2) (layer "B.Cu") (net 20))
 (segment (start 169.0688 99.06) (end 167.9056 100.2232) (width 0.2) (layer "B.Cu") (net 20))
 (segment (start 118.2138 111.18) (end 130.2788 111.18) (width 0.2) (layer "B.Cu") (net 17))
 (segment (start 117.6338 111.76) (end 118.2138 111.18) (width 0.2) (layer "B.Cu") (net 17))
 (segment (start 130.2788 111.18) (end 130.9688 110.49) (width 0.2) (layer "B.Cu") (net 17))
 (segment (start 118.7421 72.5517) (end 117.6338 73.66) (width 0.2) (layer "B.Cu") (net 2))
 (segment (start 130.9688 72.39) (end 130.8071 72.5517) (width 0.2) (layer "B.Cu") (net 2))
 (segment (start 130.8071 72.5517) (end 118.7421 72.5517) (width 0.2) (layer "B.Cu") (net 2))
 (segment (start 136.6838 111.76) (end 137.2638 111.18) (width 0.2) (layer "B.Cu") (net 3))
 (segment (start 149.3288 111.18) (end 150.0188 110.49) (width 0.2) (layer "B.Cu") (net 3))
 (segment (start 137.2638 111.18) (end 149.3288 111.18) (width 0.2) (layer "B.Cu") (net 3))
 (segment (start 156.3138 92.13) (end 168.3788 92.13) (width 0.2) (layer "B.Cu") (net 11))
 (segment (start 168.3788 92.13) (end 169.0688 91.44) (width 0.2) (layer "B.Cu") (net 11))
 (segment (start 155.7338 92.71) (end 156.3138 92.13) (width 0.2) (layer "B.Cu") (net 11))
 (segment (start 155.7338 111.76) (end 156.3138 111.18) (width 0.2) (layer "B.Cu") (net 10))
 (segment (start 156.3138 111.18) (end 168.3788 111.18) (width 0.2) (layer "B.Cu") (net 10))
 (segment (start 168.3788 111.18) (end 169.0688 110.49) (width 0.2) (layer "B.Cu") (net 10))
 (segment (start 167.62 73.87) (end 169.05 73.87) (width 0.2) (layer "B.Cu") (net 9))
 (segment (start 169.05 73.87) (end 170.49 72.43) (width 0.2) (layer "B.Cu") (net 9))
 (segment (start 112.9888 59.8487) (end 113.8238 59.8487) (width 0.2) (layer "F.Cu") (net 13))
 (segment (start 130.1656 59.4461) (end 129.4398 58.7203) (width 0.2) (layer "B.Cu") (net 13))
 (segment (start 130.1656 60.2831) (end 130.1656 59.4461) (width 0.2) (layer "B.Cu") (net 13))
 (segment (start 133.975 53.985) (end 132.8233 53.985) (width 0.2) (layer "B.Cu") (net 13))
 (segment (start 127.9914 54.2951) (end 128.6054 53.6811) (width 0.2) (layer "B.Cu") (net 13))
 (segment (start 129.4398 58.7203) (end 128.9362 58.7203) (width 0.2) (layer "B.Cu") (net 13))
 (segment (start 128.6054 53.6811) (end 132.5194 53.6811) (width 0.2) (layer "B.Cu") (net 13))
 (segment (start 127.9914 57.7755) (end 127.9914 54.2951) (width 0.2) (layer "B.Cu") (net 13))
 (segment (start 113.8238 59.8487) (end 114.9154 60.9403) (width 0.2) (layer "B.Cu") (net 13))
 (segment (start 129.5084 60.9403) (end 130.1656 60.2831) (width 0.2) (layer "B.Cu") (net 13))
 (segment (start 114.9154 60.9403) (end 129.5084 60.9403) (width 0.2) (layer "B.Cu") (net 13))
 (segment (start 128.9362 58.7203) (end 127.9914 57.7755) (width 0.2) (layer "B.Cu") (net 13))
 (segment (start 132.5194 53.6811) (end 132.8233 53.985) (width 0.2) (layer "B.Cu") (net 13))
 (segment (start 112.9888 57.3087) (end 113.8238 57.3087) (width 0.2) (layer "F.Cu") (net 14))
 (segment (start 119.9914 51.1411) (end 132.5194 51.1411) (width 0.2) (layer "B.Cu") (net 14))
 (segment (start 133.975 51.445) (end 132.8233 51.445) (width 0.2) (layer "B.Cu") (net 14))
 (segment (start 132.5194 51.1411) (end 132.8233 51.445) (width 0.2) (layer "B.Cu") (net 14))
 (segment (start 113.8238 57.3087) (end 119.9914 51.1411) (width 0.2) (layer "B.Cu") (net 14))
 (segment (start 124.797 108.4068) (end 123.9838 109.22) (width 0.2) (layer "F.Cu") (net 1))
 (segment (start 112.9888 49.6887) (end 113.8238 49.6887) (width 0.2) (layer "F.Cu") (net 1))
 (segment (start 124.797 88.1492) (end 125.4138 88.766) (width 0.2) (layer "F.Cu") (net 1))
 (segment (start 124.797 71.9332) (end 124.797 88.1492) (width 0.2) (layer "F.Cu") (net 1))
 (segment (start 123.9838 59.8487) (end 123.9838 71.12) (width 0.2) (layer "F.Cu") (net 1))
 (segment (start 123.9838 71.12) (end 124.797 71.9332) (width 0.2) (layer "F.Cu") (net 1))
 (segment (start 113.8238 49.6887) (end 123.9838 59.8487) (width 0.2) (layer "F.Cu") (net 1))
 (segment (start 124.797 91.8968) (end 124.797 108.4068) (width 0.2) (layer "F.Cu") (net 1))
 (segment (start 125.4138 91.28) (end 124.797 91.8968) (width 0.2) (layer "F.Cu") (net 1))
 (segment (start 125.4138 88.766) (end 125.4138 91.28) (width 0.2) (layer "F.Cu") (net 1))
 (segment (start 123.9838 109.22) (end 143.0338 109.22) (width 0.2) (layer "B.Cu") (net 1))
 (segment (start 129.0638 57.3087) (end 129.8988 57.3087) (width 0.2) (layer "F.Cu") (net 6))
 (segment (start 146.2929 67.0429) (end 151.8183 72.5683) (width 0.2) (layer "B.Cu") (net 6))
 (segment (start 129.0638 57.3087) (end 138.798 67.0429) (width 0.2) (layer "B.Cu") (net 6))
 (segment (start 151.8183 72.5683) (end 151.8183 73.87) (width 0.2) (layer "B.Cu") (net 6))
 (segment (start 153.12 73.87) (end 151.8183 73.87) (width 0.2) (layer "B.Cu") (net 6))
 (segment (start 138.798 67.0429) (end 146.2929 67.0429) (width 0.2) (layer "B.Cu") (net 6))
 (segment (start 151.1946 76.9446) (end 151.1946 57.4079) (width 0.2) (layer "F.Cu") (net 7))
 (segment (start 129.0638 54.7687) (end 129.8988 54.7687) (width 0.2) (layer "F.Cu") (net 7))
 (segment (start 153.12 78.87) (end 151.1946 76.9446) (width 0.2) (layer "F.Cu") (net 7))
 (via (at 151.1946 57.4079) (size 0.6) (drill 0.3) (layers "F.Cu" "B.Cu") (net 7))
 (segment (start 149.0417 55.255) (end 129.5501 55.255) (width 0.2) (layer "B.Cu") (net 7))
 (segment (start 129.5501 55.255) (end 129.0638 54.7687) (width 0.2) (layer "B.Cu") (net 7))
 (segment (start 151.1946 57.4079) (end 149.0417 55.255) (width 0.2) (layer "B.Cu") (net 7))
 (segment (start 113.4063 52.2287) (end 113.4476 52.2287) (width 0.2) (layer "F.Cu") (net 4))
 (segment (start 162.1346 90.2208) (end 162.1346 91.5604) (width 0.2) (layer "F.Cu") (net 4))
 (segment (start 118.8571 74.8613) (end 118.8571 85.0433) (width 0.2) (layer "F.Cu") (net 4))
 (segment (start 162.0838 90.17) (end 162.1346 90.2208) (width 0.2) (layer "F.Cu") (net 4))
 (segment (start 113.8238 52.2287) (end 119.088 57.4929) (width 0.2) (layer "F.Cu") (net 4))
 (segment (start 119.088 57.4929) (end 119.088 74.6304) (width 0.2) (layer "F.Cu") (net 4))
 (segment (start 162.1346 91.5604) (end 162.1346 84.3554) (width 0.2) (layer "F.Cu") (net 4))
 (segment (start 113.4476 52.2287) (end 113.8238 52.2287) (width 0.2) (layer "F.Cu") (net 4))
 (segment (start 119.088 74.6304) (end 118.8571 74.8613) (width 0.2) (layer "F.Cu") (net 4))
 (segment (start 162.1346 84.3554) (end 167.62 78.87) (width 0.2) (layer "F.Cu") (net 4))
 (segment (start 112.9888 52.2287) (end 113.4063 52.2287) (width 0.2) (layer "F.Cu") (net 4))
 (segment (start 118.8571 85.0433) (end 123.9838 90.17) (width 0.2) (layer "F.Cu") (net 4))
 (segment (start 162.1346 91.5604) (end 162.1346 109.1692) (width 0.2) (layer "F.Cu") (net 4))
 (segment (start 162.1346 109.1692) (end 162.0838 109.22) (width 0.2) (layer "F.Cu") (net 4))
 (segment (start 160.6284 88.7146) (end 162.0838 90.17) (width 0.2) (layer "B.Cu") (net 4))
 (segment (start 123.9838 90.17) (end 125.4392 88.7146) (width 0.2) (layer "B.Cu") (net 4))
 (segment (start 125.4392 88.7146) (end 160.6284 88.7146) (width 0.2) (layer "B.Cu") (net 4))
 (segment (start 113.8238 87.5763) (end 116.31 90.0625) (width 0.2) (layer "F.Cu") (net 19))
 (segment (start 130.9688 114.0717) (end 139.5354 105.5051) (width 0.2) (layer "F.Cu") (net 19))
 (segment (start 116.217 90.0625) (end 113.8238 87.6693) (width 0.2) (layer "F.Cu") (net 19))
 (segment (start 170.49 91.9229) (end 170.49 80.05) (width 0.2) (layer "F.Cu") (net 19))
 (segment (start 116.31 90.0625) (end 116.217 90.0625) (width 0.2) (layer "F.Cu") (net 19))
 (segment (start 113.4063 62.3887) (end 112.9888 62.3887) (width 0.2) (layer "F.Cu") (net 19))
 (segment (start 139.5354 105.5051) (end 139.5354 98.8116) (width 0.2) (layer "F.Cu") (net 19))
 (segment (start 113.8238 62.3887) (end 113.8238 87.5763) (width 0.2) (layer "F.Cu") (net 19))
 (segment (start 113.8238 62.3887) (end 113.4063 62.3887) (width 0.2) (layer "F.Cu") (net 19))
 (segment (start 171.5982 93.0311) (end 170.49 91.9229) (width 0.2) (layer "F.Cu") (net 19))
 (segment (start 130.9688 118.11) (end 130.9688 114.0717) (width 0.2) (layer "F.Cu") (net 19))
 (via (at 116.31 90.0625) (size 0.6) (drill 0.3) (layers "F.Cu" "B.Cu") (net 19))
 (via (at 171.5982 93.0311) (size 0.6) (drill 0.3) (layers "F.Cu" "B.Cu") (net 19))
 (via (at 139.5354 98.8116) (size 0.6) (drill 0.3) (layers "F.Cu" "B.Cu") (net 19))
 (segment (start 123.8544 92.5402) (end 128.675 92.5402) (width 0.2) (layer "B.Cu") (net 19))
 (segment (start 150.0188 99.06) (end 165.5693 99.06) (width 0.2) (layer "B.Cu") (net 19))
 (segment (start 139.7838 99.06) (end 150.0188 99.06) (width 0.2) (layer "B.Cu") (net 19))
 (segment (start 121.3767 90.0625) (end 123.8544 92.5402) (width 0.2) (layer "B.Cu") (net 19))
 (segment (start 165.5693 99.06) (end 171.5982 93.0311) (width 0.2) (layer "B.Cu") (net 19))
 (segment (start 139.5354 98.8116) (end 139.7838 99.06) (width 0.2) (layer "B.Cu") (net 19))
 (segment (start 116.31 90.0625) (end 121.3767 90.0625) (width 0.2) (layer "B.Cu") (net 19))
 (segment (start 134.9464 98.8116) (end 139.5354 98.8116) (width 0.2) (layer "B.Cu") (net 19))
 (segment (start 128.675 92.5402) (end 134.9464 98.8116) (width 0.2) (layer "B.Cu") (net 19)))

